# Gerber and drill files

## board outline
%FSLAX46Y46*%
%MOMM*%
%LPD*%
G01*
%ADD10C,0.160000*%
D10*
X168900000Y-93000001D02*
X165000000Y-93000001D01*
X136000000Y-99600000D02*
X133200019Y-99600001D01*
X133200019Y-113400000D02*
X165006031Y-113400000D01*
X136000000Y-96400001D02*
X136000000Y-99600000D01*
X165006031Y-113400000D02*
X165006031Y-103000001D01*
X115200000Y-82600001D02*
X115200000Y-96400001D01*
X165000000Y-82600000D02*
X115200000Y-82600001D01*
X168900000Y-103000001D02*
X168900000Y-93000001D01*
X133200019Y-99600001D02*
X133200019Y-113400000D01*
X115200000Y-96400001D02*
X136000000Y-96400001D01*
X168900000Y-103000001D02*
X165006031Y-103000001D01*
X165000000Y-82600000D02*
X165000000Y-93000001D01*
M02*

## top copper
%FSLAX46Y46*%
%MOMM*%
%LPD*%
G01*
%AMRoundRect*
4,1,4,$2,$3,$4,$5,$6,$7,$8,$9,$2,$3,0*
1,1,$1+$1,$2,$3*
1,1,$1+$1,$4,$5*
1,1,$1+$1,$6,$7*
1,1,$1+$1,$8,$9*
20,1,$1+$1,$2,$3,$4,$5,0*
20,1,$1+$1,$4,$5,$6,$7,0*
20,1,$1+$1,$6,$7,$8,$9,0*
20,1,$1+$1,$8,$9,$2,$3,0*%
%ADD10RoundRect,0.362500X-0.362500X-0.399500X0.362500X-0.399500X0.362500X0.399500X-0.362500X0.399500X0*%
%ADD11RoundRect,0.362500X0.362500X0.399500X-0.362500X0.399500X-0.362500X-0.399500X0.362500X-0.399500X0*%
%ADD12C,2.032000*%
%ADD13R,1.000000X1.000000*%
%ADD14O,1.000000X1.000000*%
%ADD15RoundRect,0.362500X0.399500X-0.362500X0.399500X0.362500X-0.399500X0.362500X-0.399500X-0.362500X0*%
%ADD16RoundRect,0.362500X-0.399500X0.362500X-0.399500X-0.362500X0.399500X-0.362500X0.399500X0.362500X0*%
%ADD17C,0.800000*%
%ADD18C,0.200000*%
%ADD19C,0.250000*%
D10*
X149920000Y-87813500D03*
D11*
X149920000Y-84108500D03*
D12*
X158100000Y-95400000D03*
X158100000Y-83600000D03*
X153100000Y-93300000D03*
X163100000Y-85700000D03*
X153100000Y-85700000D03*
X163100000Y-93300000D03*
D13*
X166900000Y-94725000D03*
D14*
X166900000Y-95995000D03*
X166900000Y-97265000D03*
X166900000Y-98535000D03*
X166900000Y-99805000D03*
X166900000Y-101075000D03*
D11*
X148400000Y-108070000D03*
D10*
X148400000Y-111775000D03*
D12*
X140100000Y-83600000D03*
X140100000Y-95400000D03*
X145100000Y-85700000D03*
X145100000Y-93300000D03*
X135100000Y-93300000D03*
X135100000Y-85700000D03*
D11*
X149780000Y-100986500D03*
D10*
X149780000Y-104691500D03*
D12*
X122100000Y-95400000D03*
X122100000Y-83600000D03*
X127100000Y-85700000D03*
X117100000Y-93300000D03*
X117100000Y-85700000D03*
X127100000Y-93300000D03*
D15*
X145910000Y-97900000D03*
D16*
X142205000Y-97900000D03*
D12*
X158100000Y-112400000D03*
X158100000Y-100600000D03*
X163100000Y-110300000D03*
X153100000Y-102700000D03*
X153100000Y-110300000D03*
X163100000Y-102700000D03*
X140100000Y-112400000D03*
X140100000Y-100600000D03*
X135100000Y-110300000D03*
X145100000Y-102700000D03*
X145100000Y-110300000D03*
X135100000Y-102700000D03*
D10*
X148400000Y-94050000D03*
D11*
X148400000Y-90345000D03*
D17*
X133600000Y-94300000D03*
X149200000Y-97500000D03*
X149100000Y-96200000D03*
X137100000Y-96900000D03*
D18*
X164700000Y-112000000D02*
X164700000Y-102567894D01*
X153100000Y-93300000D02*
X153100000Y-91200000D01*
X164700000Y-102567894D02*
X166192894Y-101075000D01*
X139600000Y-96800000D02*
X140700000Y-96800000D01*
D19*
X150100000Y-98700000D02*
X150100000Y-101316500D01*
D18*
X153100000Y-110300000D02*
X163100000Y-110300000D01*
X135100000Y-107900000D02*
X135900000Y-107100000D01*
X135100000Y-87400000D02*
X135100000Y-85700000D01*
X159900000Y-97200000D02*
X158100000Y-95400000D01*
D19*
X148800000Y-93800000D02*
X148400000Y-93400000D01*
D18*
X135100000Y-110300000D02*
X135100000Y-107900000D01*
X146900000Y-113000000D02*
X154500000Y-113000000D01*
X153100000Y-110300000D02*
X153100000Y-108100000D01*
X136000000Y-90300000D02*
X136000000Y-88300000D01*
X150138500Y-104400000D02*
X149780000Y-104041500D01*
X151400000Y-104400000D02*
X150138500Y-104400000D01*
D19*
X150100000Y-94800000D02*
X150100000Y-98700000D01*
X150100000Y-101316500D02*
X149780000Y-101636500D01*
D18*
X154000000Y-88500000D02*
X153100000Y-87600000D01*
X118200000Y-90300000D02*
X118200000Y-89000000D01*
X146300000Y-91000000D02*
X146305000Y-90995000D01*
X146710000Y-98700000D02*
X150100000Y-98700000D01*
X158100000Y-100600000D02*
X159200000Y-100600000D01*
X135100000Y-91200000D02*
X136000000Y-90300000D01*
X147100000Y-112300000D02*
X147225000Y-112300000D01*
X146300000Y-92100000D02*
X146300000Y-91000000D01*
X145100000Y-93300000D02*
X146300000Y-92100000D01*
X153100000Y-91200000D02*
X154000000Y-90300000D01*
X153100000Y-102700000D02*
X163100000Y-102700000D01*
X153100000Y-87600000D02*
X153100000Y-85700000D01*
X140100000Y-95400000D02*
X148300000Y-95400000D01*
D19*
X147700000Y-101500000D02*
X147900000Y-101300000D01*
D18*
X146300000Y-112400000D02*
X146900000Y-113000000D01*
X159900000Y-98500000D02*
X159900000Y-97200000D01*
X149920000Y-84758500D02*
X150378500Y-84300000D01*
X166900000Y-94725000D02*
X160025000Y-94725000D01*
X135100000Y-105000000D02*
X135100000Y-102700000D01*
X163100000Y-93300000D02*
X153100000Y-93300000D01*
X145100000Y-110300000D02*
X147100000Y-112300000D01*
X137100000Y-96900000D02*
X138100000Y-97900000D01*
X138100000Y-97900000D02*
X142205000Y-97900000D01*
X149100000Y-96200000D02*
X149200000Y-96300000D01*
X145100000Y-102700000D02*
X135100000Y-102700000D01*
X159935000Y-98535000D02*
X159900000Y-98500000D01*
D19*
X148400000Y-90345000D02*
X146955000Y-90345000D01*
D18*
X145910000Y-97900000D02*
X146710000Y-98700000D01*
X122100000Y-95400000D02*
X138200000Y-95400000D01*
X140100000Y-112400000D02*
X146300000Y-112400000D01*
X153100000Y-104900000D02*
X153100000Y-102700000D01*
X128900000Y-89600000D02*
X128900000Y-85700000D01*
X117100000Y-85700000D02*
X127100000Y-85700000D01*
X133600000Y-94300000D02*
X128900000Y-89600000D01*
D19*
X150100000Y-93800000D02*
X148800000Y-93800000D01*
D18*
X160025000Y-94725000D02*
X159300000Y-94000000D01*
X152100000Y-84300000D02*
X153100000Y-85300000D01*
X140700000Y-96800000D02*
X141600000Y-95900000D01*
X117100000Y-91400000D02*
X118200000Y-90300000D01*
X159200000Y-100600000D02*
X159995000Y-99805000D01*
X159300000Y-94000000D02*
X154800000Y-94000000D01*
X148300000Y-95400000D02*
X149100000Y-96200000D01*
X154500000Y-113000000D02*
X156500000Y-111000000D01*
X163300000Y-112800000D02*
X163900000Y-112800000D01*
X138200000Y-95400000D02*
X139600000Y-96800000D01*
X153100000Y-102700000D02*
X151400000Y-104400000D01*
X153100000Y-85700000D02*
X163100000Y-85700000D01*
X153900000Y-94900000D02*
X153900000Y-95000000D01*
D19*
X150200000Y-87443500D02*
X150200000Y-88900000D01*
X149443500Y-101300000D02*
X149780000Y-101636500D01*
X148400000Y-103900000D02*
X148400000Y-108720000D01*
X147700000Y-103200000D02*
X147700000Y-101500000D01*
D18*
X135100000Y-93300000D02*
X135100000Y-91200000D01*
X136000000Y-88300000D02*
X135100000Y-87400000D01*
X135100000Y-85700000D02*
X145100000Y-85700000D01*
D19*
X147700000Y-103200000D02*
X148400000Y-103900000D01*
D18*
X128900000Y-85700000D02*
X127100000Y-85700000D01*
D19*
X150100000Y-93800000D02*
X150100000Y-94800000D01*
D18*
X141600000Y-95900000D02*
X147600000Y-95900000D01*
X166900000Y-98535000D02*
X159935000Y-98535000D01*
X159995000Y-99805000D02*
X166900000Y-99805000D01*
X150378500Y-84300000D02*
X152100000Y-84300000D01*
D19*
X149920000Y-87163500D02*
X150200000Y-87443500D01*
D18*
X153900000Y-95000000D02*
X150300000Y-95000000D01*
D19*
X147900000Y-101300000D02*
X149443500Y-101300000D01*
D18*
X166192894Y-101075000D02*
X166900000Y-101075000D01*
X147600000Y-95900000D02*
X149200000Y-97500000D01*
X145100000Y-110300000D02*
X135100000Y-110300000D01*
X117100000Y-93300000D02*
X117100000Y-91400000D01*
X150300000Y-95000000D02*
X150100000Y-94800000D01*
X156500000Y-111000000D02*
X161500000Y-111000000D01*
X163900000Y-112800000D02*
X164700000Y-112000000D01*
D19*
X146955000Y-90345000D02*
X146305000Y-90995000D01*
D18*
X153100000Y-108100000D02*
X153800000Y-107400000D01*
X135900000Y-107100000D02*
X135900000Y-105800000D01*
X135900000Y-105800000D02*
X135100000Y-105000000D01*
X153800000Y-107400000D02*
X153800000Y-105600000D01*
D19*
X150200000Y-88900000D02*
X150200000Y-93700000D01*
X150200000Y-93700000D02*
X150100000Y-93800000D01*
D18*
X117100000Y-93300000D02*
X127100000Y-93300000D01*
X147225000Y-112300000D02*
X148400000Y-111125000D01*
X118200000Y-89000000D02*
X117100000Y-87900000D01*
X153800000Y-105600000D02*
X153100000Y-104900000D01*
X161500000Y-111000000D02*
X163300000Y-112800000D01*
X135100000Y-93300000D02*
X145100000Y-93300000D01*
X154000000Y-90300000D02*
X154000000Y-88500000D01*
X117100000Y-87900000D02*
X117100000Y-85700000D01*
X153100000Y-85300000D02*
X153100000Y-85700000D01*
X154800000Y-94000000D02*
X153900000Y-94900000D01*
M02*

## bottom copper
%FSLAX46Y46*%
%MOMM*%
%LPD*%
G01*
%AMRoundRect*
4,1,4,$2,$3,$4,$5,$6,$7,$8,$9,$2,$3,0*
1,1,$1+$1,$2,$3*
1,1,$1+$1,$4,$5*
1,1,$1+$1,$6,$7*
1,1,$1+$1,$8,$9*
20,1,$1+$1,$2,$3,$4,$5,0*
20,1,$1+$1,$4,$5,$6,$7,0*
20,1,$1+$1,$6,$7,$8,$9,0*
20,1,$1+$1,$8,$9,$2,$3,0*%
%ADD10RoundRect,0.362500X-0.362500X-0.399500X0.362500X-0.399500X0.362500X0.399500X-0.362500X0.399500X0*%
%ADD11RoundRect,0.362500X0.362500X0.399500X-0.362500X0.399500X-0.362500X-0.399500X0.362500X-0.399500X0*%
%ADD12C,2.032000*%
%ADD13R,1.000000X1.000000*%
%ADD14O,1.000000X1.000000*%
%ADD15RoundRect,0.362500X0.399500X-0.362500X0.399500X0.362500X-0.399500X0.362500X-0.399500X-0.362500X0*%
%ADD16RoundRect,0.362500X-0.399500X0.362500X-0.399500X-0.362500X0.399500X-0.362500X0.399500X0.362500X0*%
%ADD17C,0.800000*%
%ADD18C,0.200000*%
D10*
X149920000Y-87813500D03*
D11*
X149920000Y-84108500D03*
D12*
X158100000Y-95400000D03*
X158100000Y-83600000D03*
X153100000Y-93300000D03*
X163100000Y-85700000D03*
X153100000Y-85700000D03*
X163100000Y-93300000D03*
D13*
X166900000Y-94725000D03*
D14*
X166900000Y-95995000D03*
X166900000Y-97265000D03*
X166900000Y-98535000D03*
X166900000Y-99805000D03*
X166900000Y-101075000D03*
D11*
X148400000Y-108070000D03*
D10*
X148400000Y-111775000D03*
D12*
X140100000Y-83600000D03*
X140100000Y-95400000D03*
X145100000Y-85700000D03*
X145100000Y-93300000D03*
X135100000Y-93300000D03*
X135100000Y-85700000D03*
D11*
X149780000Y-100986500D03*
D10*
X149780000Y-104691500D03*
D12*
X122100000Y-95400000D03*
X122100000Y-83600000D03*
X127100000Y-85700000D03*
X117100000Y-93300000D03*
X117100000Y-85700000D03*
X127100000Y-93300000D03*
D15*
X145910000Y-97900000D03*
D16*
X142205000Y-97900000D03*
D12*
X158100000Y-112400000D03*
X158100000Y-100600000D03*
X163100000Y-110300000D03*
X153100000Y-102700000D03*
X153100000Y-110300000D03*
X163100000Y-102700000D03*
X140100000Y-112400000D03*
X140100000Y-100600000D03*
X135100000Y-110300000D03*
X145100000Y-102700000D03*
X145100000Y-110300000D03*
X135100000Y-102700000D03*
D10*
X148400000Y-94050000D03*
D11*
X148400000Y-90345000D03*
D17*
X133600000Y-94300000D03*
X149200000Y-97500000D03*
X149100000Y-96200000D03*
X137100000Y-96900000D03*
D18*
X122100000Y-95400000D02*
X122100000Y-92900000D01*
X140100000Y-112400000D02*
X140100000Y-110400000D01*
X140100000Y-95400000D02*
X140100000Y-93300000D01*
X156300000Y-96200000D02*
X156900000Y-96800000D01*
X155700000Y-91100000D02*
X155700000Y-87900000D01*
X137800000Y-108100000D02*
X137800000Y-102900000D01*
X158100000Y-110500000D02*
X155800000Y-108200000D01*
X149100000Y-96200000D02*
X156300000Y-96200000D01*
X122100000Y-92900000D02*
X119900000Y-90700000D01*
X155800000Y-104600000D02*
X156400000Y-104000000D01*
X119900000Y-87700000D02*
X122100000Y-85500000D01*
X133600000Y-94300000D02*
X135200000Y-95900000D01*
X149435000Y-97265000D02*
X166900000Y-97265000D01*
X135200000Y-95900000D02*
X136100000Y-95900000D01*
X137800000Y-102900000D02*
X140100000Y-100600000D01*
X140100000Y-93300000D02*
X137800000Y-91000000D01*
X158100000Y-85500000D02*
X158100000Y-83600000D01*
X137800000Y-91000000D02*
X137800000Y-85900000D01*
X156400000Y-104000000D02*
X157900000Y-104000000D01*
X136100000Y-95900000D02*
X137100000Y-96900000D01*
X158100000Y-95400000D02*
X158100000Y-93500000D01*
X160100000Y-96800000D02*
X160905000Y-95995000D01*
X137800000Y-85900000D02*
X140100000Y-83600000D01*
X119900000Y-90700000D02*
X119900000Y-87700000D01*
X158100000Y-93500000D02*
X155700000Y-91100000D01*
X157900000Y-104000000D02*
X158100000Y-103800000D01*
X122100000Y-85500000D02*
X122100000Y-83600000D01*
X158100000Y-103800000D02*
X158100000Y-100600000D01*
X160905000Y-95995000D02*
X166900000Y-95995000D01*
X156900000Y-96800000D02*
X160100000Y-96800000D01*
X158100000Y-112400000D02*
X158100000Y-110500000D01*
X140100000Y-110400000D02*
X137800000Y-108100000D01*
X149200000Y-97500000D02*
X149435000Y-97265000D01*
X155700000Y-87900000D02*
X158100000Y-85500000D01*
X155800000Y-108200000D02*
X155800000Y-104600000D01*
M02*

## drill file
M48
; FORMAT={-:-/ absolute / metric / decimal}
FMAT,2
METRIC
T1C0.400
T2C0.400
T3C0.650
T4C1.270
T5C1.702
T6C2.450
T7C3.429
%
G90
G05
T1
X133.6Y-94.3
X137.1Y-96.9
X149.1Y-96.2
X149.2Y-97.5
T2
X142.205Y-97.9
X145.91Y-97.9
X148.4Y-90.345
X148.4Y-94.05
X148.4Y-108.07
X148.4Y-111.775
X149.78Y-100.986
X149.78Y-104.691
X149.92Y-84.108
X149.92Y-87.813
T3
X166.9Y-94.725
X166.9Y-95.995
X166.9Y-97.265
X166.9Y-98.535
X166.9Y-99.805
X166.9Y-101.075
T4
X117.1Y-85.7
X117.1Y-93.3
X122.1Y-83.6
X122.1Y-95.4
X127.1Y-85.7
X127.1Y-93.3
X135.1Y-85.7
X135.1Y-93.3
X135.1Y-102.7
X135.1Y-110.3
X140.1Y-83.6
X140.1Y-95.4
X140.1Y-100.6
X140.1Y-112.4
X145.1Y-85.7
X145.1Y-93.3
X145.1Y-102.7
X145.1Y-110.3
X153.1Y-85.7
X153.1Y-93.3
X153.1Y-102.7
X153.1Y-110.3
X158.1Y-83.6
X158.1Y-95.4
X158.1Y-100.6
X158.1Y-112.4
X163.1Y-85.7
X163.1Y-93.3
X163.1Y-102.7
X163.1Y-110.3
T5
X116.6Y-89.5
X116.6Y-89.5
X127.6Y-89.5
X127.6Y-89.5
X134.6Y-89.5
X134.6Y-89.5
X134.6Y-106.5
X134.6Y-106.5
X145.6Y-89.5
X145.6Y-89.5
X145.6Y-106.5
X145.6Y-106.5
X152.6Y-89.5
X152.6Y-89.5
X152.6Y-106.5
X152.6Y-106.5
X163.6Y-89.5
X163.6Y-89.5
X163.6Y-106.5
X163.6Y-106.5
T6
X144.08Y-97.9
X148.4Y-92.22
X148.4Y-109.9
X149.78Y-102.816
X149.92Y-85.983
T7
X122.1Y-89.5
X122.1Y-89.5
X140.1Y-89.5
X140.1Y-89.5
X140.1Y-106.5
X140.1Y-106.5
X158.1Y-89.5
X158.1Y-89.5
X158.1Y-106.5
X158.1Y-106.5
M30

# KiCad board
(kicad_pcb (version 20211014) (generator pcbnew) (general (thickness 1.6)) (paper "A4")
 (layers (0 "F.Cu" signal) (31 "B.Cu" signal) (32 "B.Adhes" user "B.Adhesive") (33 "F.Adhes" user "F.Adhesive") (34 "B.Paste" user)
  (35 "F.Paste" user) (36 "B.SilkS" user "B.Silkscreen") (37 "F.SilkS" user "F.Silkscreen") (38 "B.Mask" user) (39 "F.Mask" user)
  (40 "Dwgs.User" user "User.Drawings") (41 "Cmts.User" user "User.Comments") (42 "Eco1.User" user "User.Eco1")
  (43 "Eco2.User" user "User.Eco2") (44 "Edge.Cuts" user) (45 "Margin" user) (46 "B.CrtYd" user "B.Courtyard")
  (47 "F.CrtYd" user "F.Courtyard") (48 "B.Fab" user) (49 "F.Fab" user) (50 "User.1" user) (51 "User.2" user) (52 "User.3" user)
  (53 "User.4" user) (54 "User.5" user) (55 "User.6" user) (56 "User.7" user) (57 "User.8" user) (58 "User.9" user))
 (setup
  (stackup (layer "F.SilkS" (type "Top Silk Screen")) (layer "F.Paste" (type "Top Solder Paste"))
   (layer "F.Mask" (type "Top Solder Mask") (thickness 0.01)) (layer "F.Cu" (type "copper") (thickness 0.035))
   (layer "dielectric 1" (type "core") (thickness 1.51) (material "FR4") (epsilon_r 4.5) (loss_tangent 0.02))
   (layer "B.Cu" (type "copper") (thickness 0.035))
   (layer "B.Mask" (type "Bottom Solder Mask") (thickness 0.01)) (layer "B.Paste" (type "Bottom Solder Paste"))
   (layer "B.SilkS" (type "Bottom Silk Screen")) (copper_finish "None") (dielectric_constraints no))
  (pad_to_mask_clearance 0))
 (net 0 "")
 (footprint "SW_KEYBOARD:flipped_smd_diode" (layer "F.Cu") (at 149.92 89.0035)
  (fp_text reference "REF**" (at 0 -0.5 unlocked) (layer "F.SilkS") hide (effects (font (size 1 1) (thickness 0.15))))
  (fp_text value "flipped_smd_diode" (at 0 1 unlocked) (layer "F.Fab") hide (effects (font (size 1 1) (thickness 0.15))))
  (pad "" np_thru_hole circle (at 0 -3.02) (size 2.45 2.45) (drill 2.45) (layers *.Mask))
  (pad "0" thru_hole roundrect (at 0 -1.19) (size 1.45 1.524) (drill 0.4) (layers *.Cu *.Mask) (roundrect_rratio 0.25))
  (pad "1" thru_hole roundrect (at 0 -4.895 180) (size 1.45 1.524) (drill 0.4) (layers *.Cu *.Mask) (roundrect_rratio 0.25)))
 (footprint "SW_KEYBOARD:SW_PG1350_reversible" (layer "F.Cu") (at 158.1 89.5)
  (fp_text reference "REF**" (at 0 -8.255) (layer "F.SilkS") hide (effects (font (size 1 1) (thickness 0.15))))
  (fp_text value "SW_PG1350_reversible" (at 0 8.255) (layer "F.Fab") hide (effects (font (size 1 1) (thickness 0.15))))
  (pad "" np_thru_hole circle (at 0 0 180) (size 3.429 3.429) (drill 3.429) (layers *.Cu *.Mask))
  (pad "" np_thru_hole circle (at 5.5 0) (size 1.7018 1.7018) (drill 1.7018) (layers *.Cu *.Mask))
  (pad "" np_thru_hole circle (at 5.5 0 180) (size 1.7018 1.7018) (drill 1.7018) (layers *.Cu *.Mask))
  (pad "" np_thru_hole circle (at -5.5 0) (size 1.7018 1.7018) (drill 1.7018) (layers *.Cu *.Mask))
  (pad "" np_thru_hole circle (at 0 0) (size 3.429 3.429) (drill 3.429) (layers *.Cu *.Mask))
  (pad "" np_thru_hole circle (at -5.5 0 180) (size 1.7018 1.7018) (drill 1.7018) (layers *.Cu *.Mask))
  (pad "1" thru_hole circle (at 0 5.9) (size 2.032 2.032) (drill 1.27) (layers *.Cu *.Mask))
  (pad "1" thru_hole circle (at 0 -5.9 180) (size 2.032 2.032) (drill 1.27) (layers *.Cu *.Mask))
  (pad "2" thru_hole circle (at -5 3.8) (size 2.032 2.032) (drill 1.27) (layers *.Cu *.Mask))
  (pad "2" thru_hole circle (at 5 -3.8 180) (size 2.032 2.032) (drill 1.27) (layers *.Cu *.Mask))
  (pad "2" thru_hole circle (at -5 -3.8 180) (size 2.032 2.032) (drill 1.27) (layers *.Cu *.Mask))
  (pad "2" thru_hole circle (at 5 3.8) (size 2.032 2.032) (drill 1.27) (layers *.Cu *.Mask)))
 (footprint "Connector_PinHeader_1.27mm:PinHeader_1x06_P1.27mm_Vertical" (layer "F.Cu") (at 166.9 94.725)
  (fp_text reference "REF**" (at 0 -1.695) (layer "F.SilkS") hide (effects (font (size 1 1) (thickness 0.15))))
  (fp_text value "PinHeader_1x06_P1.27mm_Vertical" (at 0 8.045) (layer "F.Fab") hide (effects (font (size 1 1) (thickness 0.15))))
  (pad "1" thru_hole rect (at 0 0) (size 1 1) (drill 0.65) (layers *.Cu *.Mask))
  (pad "2" thru_hole oval (at 0 1.27) (size 1 1) (drill 0.65) (layers *.Cu *.Mask))
  (pad "3" thru_hole oval (at 0 2.54) (size 1 1) (drill 0.65) (layers *.Cu *.Mask))
  (pad "4" thru_hole oval (at 0 3.81) (size 1 1) (drill 0.65) (layers *.Cu *.Mask))
  (pad "5" thru_hole oval (at 0 5.08) (size 1 1) (drill 0.65) (layers *.Cu *.Mask))
  (pad "6" thru_hole oval (at 0 6.35) (size 1 1) (drill 0.65) (layers *.Cu *.Mask)))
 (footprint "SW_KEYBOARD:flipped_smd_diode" (layer "F.Cu") (at 148.4 106.88 180)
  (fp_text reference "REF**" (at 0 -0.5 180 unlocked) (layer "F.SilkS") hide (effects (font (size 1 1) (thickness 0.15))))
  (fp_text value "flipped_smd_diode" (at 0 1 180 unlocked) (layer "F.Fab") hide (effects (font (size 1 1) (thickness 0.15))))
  (pad "" np_thru_hole circle (at 0 -3.02 180) (size 2.45 2.45) (drill 2.45) (layers *.Mask))
  (pad "0" thru_hole roundrect (at 0 -1.19 180) (size 1.45 1.524) (drill 0.4) (layers *.Cu *.Mask) (roundrect_rratio 0.25))
  (pad "1" thru_hole roundrect (at 0 -4.895) (size 1.45 1.524) (drill 0.4) (layers *.Cu *.Mask) (roundrect_rratio 0.25)))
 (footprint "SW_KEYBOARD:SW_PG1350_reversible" (layer "F.Cu") (at 140.1 89.5)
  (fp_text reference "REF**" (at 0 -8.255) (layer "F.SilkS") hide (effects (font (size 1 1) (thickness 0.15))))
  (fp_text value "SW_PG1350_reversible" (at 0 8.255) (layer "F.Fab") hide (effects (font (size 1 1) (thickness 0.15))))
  (pad "" np_thru_hole circle (at 0 0 180) (size 3.429 3.429) (drill 3.429) (layers *.Cu *.Mask))
  (pad "" np_thru_hole circle (at 5.5 0 180) (size 1.7018 1.7018) (drill 1.7018) (layers *.Cu *.Mask))
  (pad "" np_thru_hole circle (at -5.5 0) (size 1.7018 1.7018) (drill 1.7018) (layers *.Cu *.Mask))
  (pad "" np_thru_hole circle (at 0 0) (size 3.429 3.429) (drill 3.429) (layers *.Cu *.Mask))
  (pad "" np_thru_hole circle (at 5.5 0) (size 1.7018 1.7018) (drill 1.7018) (layers *.Cu *.Mask))
  (pad "" np_thru_hole circle (at -5.5 0 180) (size 1.7018 1.7018) (drill 1.7018) (layers *.Cu *.Mask))
  (pad "1" thru_hole circle (at 0 -5.9 180) (size 2.032 2.032) (drill 1.27) (layers *.Cu *.Mask))
  (pad "1" thru_hole circle (at 0 5.9) (size 2.032 2.032) (drill 1.27) (layers *.Cu *.Mask))
  (pad "2" thru_hole circle (at 5 -3.8 180) (size 2.032 2.032) (drill 1.27) (layers *.Cu *.Mask))
  (pad "2" thru_hole circle (at 5 3.8) (size 2.032 2.032) (drill 1.27) (layers *.Cu *.Mask))
  (pad "2" thru_hole circle (at -5 3.8) (size 2.032 2.032) (drill 1.27) (layers *.Cu *.Mask))
  (pad "2" thru_hole circle (at -5 -3.8 180) (size 2.032 2.032) (drill 1.27) (layers *.Cu *.Mask)))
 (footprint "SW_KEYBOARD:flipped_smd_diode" (layer "F.Cu") (at 149.78 99.7965 180)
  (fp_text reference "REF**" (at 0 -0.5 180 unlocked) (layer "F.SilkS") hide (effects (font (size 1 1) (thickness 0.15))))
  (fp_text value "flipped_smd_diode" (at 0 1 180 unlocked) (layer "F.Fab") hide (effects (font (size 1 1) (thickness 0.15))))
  (pad "" np_thru_hole circle (at 0 -3.02 180) (size 2.45 2.45) (drill 2.45) (layers *.Mask))
  (pad "0" thru_hole roundrect (at 0 -1.19 180) (size 1.45 1.524) (drill 0.4) (layers *.Cu *.Mask) (roundrect_rratio 0.25))
  (pad "1" thru_hole roundrect (at 0 -4.895) (size 1.45 1.524) (drill 0.4) (layers *.Cu *.Mask) (roundrect_rratio 0.25)))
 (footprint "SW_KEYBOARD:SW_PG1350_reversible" (layer "F.Cu") (at 122.1 89.5)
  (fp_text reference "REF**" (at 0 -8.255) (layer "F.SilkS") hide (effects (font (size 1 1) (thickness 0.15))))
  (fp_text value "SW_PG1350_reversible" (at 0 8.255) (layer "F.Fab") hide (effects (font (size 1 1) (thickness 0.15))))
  (pad "" np_thru_hole circle (at 0 0 180) (size 3.429 3.429) (drill 3.429) (layers *.Cu *.Mask))
  (pad "" np_thru_hole circle (at 0 0) (size 3.429 3.429) (drill 3.429) (layers *.Cu *.Mask))
  (pad "" np_thru_hole circle (at 5.5 0) (size 1.7018 1.7018) (drill 1.7018) (layers *.Cu *.Mask))
  (pad "" np_thru_hole circle (at -5.5 0) (size 1.7018 1.7018) (drill 1.7018) (layers *.Cu *.Mask))
  (pad "" np_thru_hole circle (at 5.5 0 180) (size 1.7018 1.7018) (drill 1.7018) (layers *.Cu *.Mask))
  (pad "" np_thru_hole circle (at -5.5 0 180) (size 1.7018 1.7018) (drill 1.7018) (layers *.Cu *.Mask))
  (pad "1" thru_hole circle (at 0 5.9) (size 2.032 2.032) (drill 1.27) (layers *.Cu *.Mask))
  (pad "1" thru_hole circle (at 0 -5.9 180) (size 2.032 2.032) (drill 1.27) (layers *.Cu *.Mask))
  (pad "2" thru_hole circle (at 5 -3.8 180) (size 2.032 2.032) (drill 1.27) (layers *.Cu *.Mask))
  (pad "2" thru_hole circle (at -5 3.8) (size 2.032 2.032) (drill 1.27) (layers *.Cu *.Mask))
  (pad "2" thru_hole circle (at -5 -3.8 180) (size 2.032 2.032) (drill 1.27) (layers *.Cu *.Mask))
  (pad "2" thru_hole circle (at 5 3.8) (size 2.032 2.032) (drill 1.27) (layers *.Cu *.Mask)))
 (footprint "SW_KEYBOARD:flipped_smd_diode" (layer "F.Cu") (at 147.1 97.9 90)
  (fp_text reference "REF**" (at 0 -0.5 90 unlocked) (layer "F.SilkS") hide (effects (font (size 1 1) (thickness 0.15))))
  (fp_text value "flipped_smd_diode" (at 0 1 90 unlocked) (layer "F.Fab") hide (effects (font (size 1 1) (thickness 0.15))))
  (pad "" np_thru_hole circle (at 0 -3.02 90) (size 2.45 2.45) (drill 2.45) (layers *.Mask))
  (pad "0" thru_hole roundrect (at 0 -1.19 90) (size 1.45 1.524) (drill 0.4) (layers *.Cu *.Mask) (roundrect_rratio 0.25))
  (pad "1" thru_hole roundrect (at 0 -4.895 270) (size 1.45 1.524) (drill 0.4) (layers *.Cu *.Mask) (roundrect_rratio 0.25)))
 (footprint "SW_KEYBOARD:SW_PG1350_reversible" (layer "F.Cu") (at 158.1 106.5)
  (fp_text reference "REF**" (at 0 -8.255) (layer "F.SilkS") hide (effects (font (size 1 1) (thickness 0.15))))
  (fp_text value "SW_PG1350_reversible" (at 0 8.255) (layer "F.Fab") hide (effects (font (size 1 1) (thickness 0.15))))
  (pad "" np_thru_hole circle (at 0 0 180) (size 3.429 3.429) (drill 3.429) (layers *.Cu *.Mask))
  (pad "" np_thru_hole circle (at 5.5 0) (size 1.7018 1.7018) (drill 1.7018) (layers *.Cu *.Mask))
  (pad "" np_thru_hole circle (at 5.5 0 180) (size 1.7018 1.7018) (drill 1.7018) (layers *.Cu *.Mask))
  (pad "" np_thru_hole circle (at -5.5 0 180) (size 1.7018 1.7018) (drill 1.7018) (layers *.Cu *.Mask))
  (pad "" np_thru_hole circle (at -5.5 0) (size 1.7018 1.7018) (drill 1.7018) (layers *.Cu *.Mask))
  (pad "" np_thru_hole circle (at 0 0) (size 3.429 3.429) (drill 3.429) (layers *.Cu *.Mask))
  (pad "1" thru_hole circle (at 0 5.9) (size 2.032 2.032) (drill 1.27) (layers *.Cu *.Mask))
  (pad "1" thru_hole circle (at 0 -5.9 180) (size 2.032 2.032) (drill 1.27) (layers *.Cu *.Mask))
  (pad "2" thru_hole circle (at 5 3.8) (size 2.032 2.032) (drill 1.27) (layers *.Cu *.Mask))
  (pad "2" thru_hole circle (at -5 -3.8 180) (size 2.032 2.032) (drill 1.27) (layers *.Cu *.Mask))
  (pad "2" thru_hole circle (at -5 3.8) (size 2.032 2.032) (drill 1.27) (layers *.Cu *.Mask))
  (pad "2" thru_hole circle (at 5 -3.8 180) (size 2.032 2.032) (drill 1.27) (layers *.Cu *.Mask)))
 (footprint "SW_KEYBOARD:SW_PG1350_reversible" (layer "F.Cu") (at 140.1 106.5)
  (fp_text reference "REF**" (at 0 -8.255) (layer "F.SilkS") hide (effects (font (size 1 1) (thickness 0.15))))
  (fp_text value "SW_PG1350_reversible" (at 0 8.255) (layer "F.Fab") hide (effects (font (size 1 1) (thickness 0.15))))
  (pad "" np_thru_hole circle (at 5.5 0 180) (size 1.7018 1.7018) (drill 1.7018) (layers *.Cu *.Mask))
  (pad "" np_thru_hole circle (at -5.5 0 180) (size 1.7018 1.7018) (drill 1.7018) (layers *.Cu *.Mask))
  (pad "" np_thru_hole circle (at 0 0 180) (size 3.429 3.429) (drill 3.429) (layers *.Cu *.Mask))
  (pad "" np_thru_hole circle (at 5.5 0) (size 1.7018 1.7018) (drill 1.7018) (layers *.Cu *.Mask))
  (pad "" np_thru_hole circle (at -5.5 0) (size 1.7018 1.7018) (drill 1.7018) (layers *.Cu *.Mask))
  (pad "" np_thru_hole circle (at 0 0) (size 3.429 3.429) (drill 3.429) (layers *.Cu *.Mask))
  (pad "1" thru_hole circle (at 0 5.9) (size 2.032 2.032) (drill 1.27) (layers *.Cu *.Mask))
  (pad "1" thru_hole circle (at 0 -5.9 180) (size 2.032 2.032) (drill 1.27) (layers *.Cu *.Mask))
  (pad "2" thru_hole circle (at -5 3.8) (size 2.032 2.032) (drill 1.27) (layers *.Cu *.Mask))
  (pad "2" thru_hole circle (at 5 -3.8 180) (size 2.032 2.032) (drill 1.27) (layers *.Cu *.Mask))
  (pad "2" thru_hole circle (at 5 3.8) (size 2.032 2.032) (drill 1.27) (layers *.Cu *.Mask))
  (pad "2" thru_hole circle (at -5 -3.8 180) (size 2.032 2.032) (drill 1.27) (layers *.Cu *.Mask)))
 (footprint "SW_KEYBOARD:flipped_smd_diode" (layer "F.Cu") (at 148.4 95.24)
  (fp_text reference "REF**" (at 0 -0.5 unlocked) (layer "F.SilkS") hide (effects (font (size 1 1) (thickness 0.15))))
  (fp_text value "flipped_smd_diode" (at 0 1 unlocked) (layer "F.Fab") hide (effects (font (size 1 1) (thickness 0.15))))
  (pad "" np_thru_hole circle (at 0 -3.02) (size 2.45 2.45) (drill 2.45) (layers *.Mask))
  (pad "0" thru_hole roundrect (at 0 -1.19) (size 1.45 1.524) (drill 0.4) (layers *.Cu *.Mask) (roundrect_rratio 0.25))
  (pad "1" thru_hole roundrect (at 0 -4.895 180) (size 1.45 1.524) (drill 0.4) (layers *.Cu *.Mask) (roundrect_rratio 0.25)))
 (gr_line (start 168.9 93.000001) (end 165 93.000001) (layer "Edge.Cuts") (width 0.16))
 (gr_line (start 136 99.6) (end 133.200019 99.600001) (layer "Edge.Cuts") (width 0.16))
 (gr_line (start 133.200019 113.4) (end 165.006031 113.4) (layer "Edge.Cuts") (width 0.16))
 (gr_line (start 136 96.400001) (end 136 99.6) (layer "Edge.Cuts") (width 0.16))
 (gr_line (start 165.006031 113.4) (end 165.006031 103.000001) (layer "Edge.Cuts") (width 0.16))
 (gr_line (start 115.2 82.600001) (end 115.2 96.400001) (layer "Edge.Cuts") (width 0.16))
 (gr_line (start 165 82.6) (end 115.2 82.600001) (layer "Edge.Cuts") (width 0.16))
 (gr_line (start 168.9 103.000001) (end 168.9 93.000001) (layer "Edge.Cuts") (width 0.16))
 (gr_line (start 133.200019 99.600001) (end 133.200019 113.4) (layer "Edge.Cuts") (width 0.16))
 (gr_line (start 115.2 96.400001) (end 136 96.400001) (layer "Edge.Cuts") (width 0.16))
 (gr_line (start 168.9 103.000001) (end 165.006031 103.000001) (layer "Edge.Cuts") (width 0.16))
 (gr_line (start 165 82.6) (end 165 93.000001) (layer "Edge.Cuts") (width 0.16))
 (segment (start 164.7 112) (end 164.7 102.567894) (width 0.2) (layer "F.Cu") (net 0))
 (segment (start 153.1 93.3) (end 153.1 91.2) (width 0.2) (layer "F.Cu") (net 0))
 (segment (start 164.7 102.567894) (end 166.192894 101.075) (width 0.2) (layer "F.Cu") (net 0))
 (segment (start 139.6 96.8) (end 140.7 96.8) (width 0.2) (layer "F.Cu") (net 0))
 (segment (start 150.1 98.7) (end 150.1 101.3165) (width 0.25) (layer "F.Cu") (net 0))
 (segment (start 153.1 110.3) (end 163.1 110.3) (width 0.2) (layer "F.Cu") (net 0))
 (segment (start 135.1 107.9) (end 135.9 107.1) (width 0.2) (layer "F.Cu") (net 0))
 (segment (start 135.1 87.4) (end 135.1 85.7) (width 0.2) (layer "F.Cu") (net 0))
 (segment (start 159.9 97.2) (end 158.1 95.4) (width 0.2) (layer "F.Cu") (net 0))
 (segment (start 148.8 93.8) (end 148.4 93.4) (width 0.25) (layer "F.Cu") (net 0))
 (segment (start 135.1 110.3) (end 135.1 107.9) (width 0.2) (layer "F.Cu") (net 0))
 (segment (start 146.9 113) (end 154.5 113) (width 0.2) (layer "F.Cu") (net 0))
 (segment (start 153.1 110.3) (end 153.1 108.1) (width 0.2) (layer "F.Cu") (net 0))
 (segment (start 136 90.3) (end 136 88.3) (width 0.2) (layer "F.Cu") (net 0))
 (segment (start 150.1385 104.4) (end 149.78 104.0415) (width 0.2) (layer "F.Cu") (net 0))
 (segment (start 151.4 104.4) (end 150.1385 104.4) (width 0.2) (layer "F.Cu") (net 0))
 (segment (start 150.1 94.8) (end 150.1 98.7) (width 0.25) (layer "F.Cu") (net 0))
 (segment (start 150.1 101.3165) (end 149.78 101.6365) (width 0.25) (layer "F.Cu") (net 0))
 (segment (start 154 88.5) (end 153.1 87.6) (width 0.2) (layer "F.Cu") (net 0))
 (segment (start 118.2 90.3) (end 118.2 89) (width 0.2) (layer "F.Cu") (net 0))
 (segment (start 146.3 91) (end 146.305 90.995) (width 0.2) (layer "F.Cu") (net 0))
 (segment (start 146.71 98.7) (end 150.1 98.7) (width 0.2) (layer "F.Cu") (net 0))
 (segment (start 158.1 100.6) (end 159.2 100.6) (width 0.2) (layer "F.Cu") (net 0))
 (segment (start 135.1 91.2) (end 136 90.3) (width 0.2) (layer "F.Cu") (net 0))
 (segment (start 147.1 112.3) (end 147.225 112.3) (width 0.2) (layer "F.Cu") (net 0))
 (segment (start 146.3 92.1) (end 146.3 91) (width 0.2) (layer "F.Cu") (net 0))
 (segment (start 145.1 93.3) (end 146.3 92.1) (width 0.2) (layer "F.Cu") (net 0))
 (segment (start 153.1 91.2) (end 154 90.3) (width 0.2) (layer "F.Cu") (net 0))
 (segment (start 153.1 102.7) (end 163.1 102.7) (width 0.2) (layer "F.Cu") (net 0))
 (segment (start 153.1 87.6) (end 153.1 85.7) (width 0.2) (layer "F.Cu") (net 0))
 (segment (start 140.1 95.4) (end 148.3 95.4) (width 0.2) (layer "F.Cu") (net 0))
 (segment (start 147.7 101.5) (end 147.9 101.3) (width 0.25) (layer "F.Cu") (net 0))
 (segment (start 146.3 112.4) (end 146.9 113) (width 0.2) (layer "F.Cu") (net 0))
 (segment (start 159.9 98.5) (end 159.9 97.2) (width 0.2) (layer "F.Cu") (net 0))
 (segment (start 149.92 84.7585) (end 150.3785 84.3) (width 0.2) (layer "F.Cu") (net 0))
 (segment (start 166.9 94.725) (end 160.025 94.725) (width 0.2) (layer "F.Cu") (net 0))
 (segment (start 135.1 105) (end 135.1 102.7) (width 0.2) (layer "F.Cu") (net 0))
 (segment (start 163.1 93.3) (end 153.1 93.3) (width 0.2) (layer "F.Cu") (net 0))
 (segment (start 145.1 110.3) (end 147.1 112.3) (width 0.2) (layer "F.Cu") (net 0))
 (segment (start 137.1 96.9) (end 138.1 97.9) (width 0.2) (layer "F.Cu") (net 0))
 (segment (start 138.1 97.9) (end 142.205 97.9) (width 0.2) (layer "F.Cu") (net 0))
 (segment (start 149.1 96.2) (end 149.2 96.3) (width 0.2) (layer "F.Cu") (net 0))
 (segment (start 145.1 102.7) (end 135.1 102.7) (width 0.2) (layer "F.Cu") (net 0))
 (segment (start 159.935 98.535) (end 159.9 98.5) (width 0.2) (layer "F.Cu") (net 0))
 (segment (start 148.4 90.345) (end 146.955 90.345) (width 0.25) (layer "F.Cu") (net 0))
 (segment (start 145.91 97.9) (end 146.71 98.7) (width 0.2) (layer "F.Cu") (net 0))
 (segment (start 122.1 95.4) (end 138.2 95.4) (width 0.2) (layer "F.Cu") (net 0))
 (segment (start 140.1 112.4) (end 146.3 112.4) (width 0.2) (layer "F.Cu") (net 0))
 (segment (start 153.1 104.9) (end 153.1 102.7) (width 0.2) (layer "F.Cu") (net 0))
 (segment (start 128.9 89.6) (end 128.9 85.7) (width 0.2) (layer "F.Cu") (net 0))
 (segment (start 117.1 85.7) (end 127.1 85.7) (width 0.2) (layer "F.Cu") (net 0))
 (segment (start 133.6 94.3) (end 128.9 89.6) (width 0.2) (layer "F.Cu") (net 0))
 (segment (start 150.1 93.8) (end 148.8 93.8) (width 0.25) (layer "F.Cu") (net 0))
 (segment (start 160.025 94.725) (end 159.3 94) (width 0.2) (layer "F.Cu") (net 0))
 (segment (start 152.1 84.3) (end 153.1 85.3) (width 0.2) (layer "F.Cu") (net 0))
 (segment (start 140.7 96.8) (end 141.6 95.9) (width 0.2) (layer "F.Cu") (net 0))
 (segment (start 117.1 91.4) (end 118.2 90.3) (width 0.2) (layer "F.Cu") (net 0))
 (segment (start 159.2 100.6) (end 159.995 99.805) (width 0.2) (layer "F.Cu") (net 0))
 (segment (start 159.3 94) (end 154.8 94) (width 0.2) (layer "F.Cu") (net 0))
 (segment (start 148.3 95.4) (end 149.1 96.2) (width 0.2) (layer "F.Cu") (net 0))
 (segment (start 154.5 113) (end 156.5 111) (width 0.2) (layer "F.Cu") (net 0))
 (segment (start 163.3 112.8) (end 163.9 112.8) (width 0.2) (layer "F.Cu") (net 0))
 (segment (start 138.2 95.4) (end 139.6 96.8) (width 0.2) (layer "F.Cu") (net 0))
 (segment (start 153.1 102.7) (end 151.4 104.4) (width 0.2) (layer "F.Cu") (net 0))
 (segment (start 153.1 85.7) (end 163.1 85.7) (width 0.2) (layer "F.Cu") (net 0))
 (segment (start 153.9 94.9) (end 153.9 95) (width 0.2) (layer "F.Cu") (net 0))
 (segment (start 150.2 87.4435) (end 150.2 88.9) (width 0.25) (layer "F.Cu") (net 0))
 (segment (start 149.4435 101.3) (end 149.78 101.6365) (width 0.25) (layer "F.Cu") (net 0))
 (segment (start 148.4 103.9) (end 148.4 108.72) (width 0.25) (layer "F.Cu") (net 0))
 (segment (start 147.7 103.2) (end 147.7 101.5) (width 0.25) (layer "F.Cu") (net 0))
 (segment (start 135.1 93.3) (end 135.1 91.2) (width 0.2) (layer "F.Cu") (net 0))
 (segment (start 136 88.3) (end 135.1 87.4) (width 0.2) (layer "F.Cu") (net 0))
 (segment (start 135.1 85.7) (end 145.1 85.7) (width 0.2) (layer "F.Cu") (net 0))
 (segment (start 147.7 103.2) (end 148.4 103.9) (width 0.25) (layer "F.Cu") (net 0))
 (segment (start 128.9 85.7) (end 127.1 85.7) (width 0.2) (layer "F.Cu") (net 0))
 (segment (start 150.1 93.8) (end 150.1 94.8) (width 0.25) (layer "F.Cu") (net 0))
 (segment (start 141.6 95.9) (end 147.6 95.9) (width 0.2) (layer "F.Cu") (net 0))
 (segment (start 166.9 98.535) (end 159.935 98.535) (width 0.2) (layer "F.Cu") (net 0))
 (segment (start 159.995 99.805) (end 166.9 99.805) (width 0.2) (layer "F.Cu") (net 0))
 (segment (start 150.3785 84.3) (end 152.1 84.3) (width 0.2) (layer "F.Cu") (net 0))
 (segment (start 149.92 87.1635) (end 150.2 87.4435) (width 0.25) (layer "F.Cu") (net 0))
 (segment (start 153.9 95) (end 150.3 95) (width 0.2) (layer "F.Cu") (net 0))
 (segment (start 147.9 101.3) (end 149.4435 101.3) (width 0.25) (layer "F.Cu") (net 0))
 (segment (start 166.192894 101.075) (end 166.9 101.075) (width 0.2) (layer "F.Cu") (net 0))
 (segment (start 147.6 95.9) (end 149.2 97.5) (width 0.2) (layer "F.Cu") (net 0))
 (segment (start 145.1 110.3) (end 135.1 110.3) (width 0.2) (layer "F.Cu") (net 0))
 (segment (start 117.1 93.3) (end 117.1 91.4) (width 0.2) (layer "F.Cu") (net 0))
 (segment (start 150.3 95) (end 150.1 94.8) (width 0.2) (layer "F.Cu") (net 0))
 (segment (start 156.5 111) (end 161.5 111) (width 0.2) (layer "F.Cu") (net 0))
 (segment (start 163.9 112.8) (end 164.7 112) (width 0.2) (layer "F.Cu") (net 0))
 (segment (start 146.955 90.345) (end 146.305 90.995) (width 0.25) (layer "F.Cu") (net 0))
 (segment (start 153.1 108.1) (end 153.8 107.4) (width 0.2) (layer "F.Cu") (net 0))
 (segment (start 135.9 107.1) (end 135.9 105.8) (width 0.2) (layer "F.Cu") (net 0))
 (segment (start 135.9 105.8) (end 135.1 105) (width 0.2) (layer "F.Cu") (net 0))
 (segment (start 153.8 107.4) (end 153.8 105.6) (width 0.2) (layer "F.Cu") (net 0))
 (segment (start 150.2 88.9) (end 150.2 93.7) (width 0.25) (layer "F.Cu") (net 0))
 (segment (start 150.2 93.7) (end 150.1 93.8) (width 0.25) (layer "F.Cu") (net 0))
 (segment (start 117.1 93.3) (end 127.1 93.3) (width 0.2) (layer "F.Cu") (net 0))
 (segment (start 147.225 112.3) (end 148.4 111.125) (width 0.2) (layer "F.Cu") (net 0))
 (segment (start 118.2 89) (end 117.1 87.9) (width 0.2) (layer "F.Cu") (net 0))
 (segment (start 153.8 105.6) (end 153.1 104.9) (width 0.2) (layer "F.Cu") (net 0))
 (segment (start 161.5 111) (end 163.3 112.8) (width 0.2) (layer "F.Cu") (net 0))
 (segment (start 135.1 93.3) (end 145.1 93.3) (width 0.2) (layer "F.Cu") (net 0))
 (segment (start 154 90.3) (end 154 88.5) (width 0.2) (layer "F.Cu") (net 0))
 (segment (start 117.1 87.9) (end 117.1 85.7) (width 0.2) (layer "F.Cu") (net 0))
 (segment (start 153.1 85.3) (end 153.1 85.7) (width 0.2) (layer "F.Cu") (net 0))
 (segment (start 154.8 94) (end 153.9 94.9) (width 0.2) (layer "F.Cu") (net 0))
 (via (at 133.6 94.3) (size 0.8) (drill 0.4) (layers "F.Cu" "B.Cu") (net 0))
 (via (at 149.2 97.5) (size 0.8) (drill 0.4) (layers "F.Cu" "B.Cu") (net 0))
 (via (at 149.1 96.2) (size 0.8) (drill 0.4) (layers "F.Cu" "B.Cu") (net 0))
 (via (at 137.1 96.9) (size 0.8) (drill 0.4) (layers "F.Cu" "B.Cu") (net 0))
 (segment (start 122.1 95.4) (end 122.1 92.9) (width 0.2) (layer "B.Cu") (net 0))
 (segment (start 140.1 112.4) (end 140.1 110.4) (width 0.2) (layer "B.Cu") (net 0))
 (segment (start 140.1 95.4) (end 140.1 93.3) (width 0.2) (layer "B.Cu") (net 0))
 (segment (start 156.3 96.2) (end 156.9 96.8) (width 0.2) (layer "B.Cu") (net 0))
 (segment (start 155.7 91.1) (end 155.7 87.9) (width 0.2) (layer "B.Cu") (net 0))
 (segment (start 137.8 108.1) (end 137.8 102.9) (width 0.2) (layer "B.Cu") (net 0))
 (segment (start 158.1 110.5) (end 155.8 108.2) (width 0.2) (layer "B.Cu") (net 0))
 (segment (start 149.1 96.2) (end 156.3 96.2) (width 0.2) (layer "B.Cu") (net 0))
 (segment (start 122.1 92.9) (end 119.9 90.7) (width 0.2) (layer "B.Cu") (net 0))
 (segment (start 155.8 104.6) (end 156.4 104) (width 0.2) (layer "B.Cu") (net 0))
 (segment (start 119.9 87.7) (end 122.1 85.5) (width 0.2) (layer "B.Cu") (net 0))
 (segment (start 133.6 94.3) (end 135.2 95.9) (width 0.2) (layer "B.Cu") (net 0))
 (segment (start 149.435 97.265) (end 166.9 97.265) (width 0.2) (layer "B.Cu") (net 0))
 (segment (start 135.2 95.9) (end 136.1 95.9) (width 0.2) (layer "B.Cu") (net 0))
 (segment (start 137.8 102.9) (end 140.1 100.6) (width 0.2) (layer "B.Cu") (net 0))
 (segment (start 140.1 93.3) (end 137.8 91) (width 0.2) (layer "B.Cu") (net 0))
 (segment (start 158.1 85.5) (end 158.1 83.6) (width 0.2) (layer "B.Cu") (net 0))
 (segment (start 137.8 91) (end 137.8 85.9) (width 0.2) (layer "B.Cu") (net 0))
 (segment (start 156.4 104) (end 157.9 104) (width 0.2) (layer "B.Cu") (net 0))
 (segment (start 136.1 95.9) (end 137.1 96.9) (width 0.2) (layer "B.Cu") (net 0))
 (segment (start 158.1 95.4) (end 158.1 93.5) (width 0.2) (layer "B.Cu") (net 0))
 (segment (start 160.1 96.8) (end 160.905 95.995) (width 0.2) (layer "B.Cu") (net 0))
 (segment (start 137.8 85.9) (end 140.1 83.6) (width 0.2) (layer "B.Cu") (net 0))
 (segment (start 119.9 90.7) (end 119.9 87.7) (width 0.2) (layer "B.Cu") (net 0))
 (segment (start 158.1 93.5) (end 155.7 91.1) (width 0.2) (layer "B.Cu") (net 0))
 (segment (start 157.9 104) (end 158.1 103.8) (width 0.2) (layer "B.Cu") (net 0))
 (segment (start 122.1 85.5) (end 122.1 83.6) (width 0.2) (layer "B.Cu") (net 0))
 (segment (start 158.1 103.8) (end 158.1 100.6) (width 0.2) (layer "B.Cu") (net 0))
 (segment (start 160.905 95.995) (end 166.9 95.995) (width 0.2) (layer "B.Cu") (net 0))
 (segment (start 156.9 96.8) (end 160.1 96.8) (width 0.2) (layer "B.Cu") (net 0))
 (segment (start 158.1 112.4) (end 158.1 110.5) (width 0.2) (layer "B.Cu") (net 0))
 (segment (start 140.1 110.4) (end 137.8 108.1) (width 0.2) (layer "B.Cu") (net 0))
 (segment (start 149.2 97.5) (end 149.435 97.265) (width 0.2) (layer "B.Cu") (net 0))
 (segment (start 155.7 87.9) (end 158.1 85.5) (width 0.2) (layer "B.Cu") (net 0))
 (segment (start 155.8 108.2) (end 155.8 104.6) (width 0.2) (layer "B.Cu") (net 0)))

